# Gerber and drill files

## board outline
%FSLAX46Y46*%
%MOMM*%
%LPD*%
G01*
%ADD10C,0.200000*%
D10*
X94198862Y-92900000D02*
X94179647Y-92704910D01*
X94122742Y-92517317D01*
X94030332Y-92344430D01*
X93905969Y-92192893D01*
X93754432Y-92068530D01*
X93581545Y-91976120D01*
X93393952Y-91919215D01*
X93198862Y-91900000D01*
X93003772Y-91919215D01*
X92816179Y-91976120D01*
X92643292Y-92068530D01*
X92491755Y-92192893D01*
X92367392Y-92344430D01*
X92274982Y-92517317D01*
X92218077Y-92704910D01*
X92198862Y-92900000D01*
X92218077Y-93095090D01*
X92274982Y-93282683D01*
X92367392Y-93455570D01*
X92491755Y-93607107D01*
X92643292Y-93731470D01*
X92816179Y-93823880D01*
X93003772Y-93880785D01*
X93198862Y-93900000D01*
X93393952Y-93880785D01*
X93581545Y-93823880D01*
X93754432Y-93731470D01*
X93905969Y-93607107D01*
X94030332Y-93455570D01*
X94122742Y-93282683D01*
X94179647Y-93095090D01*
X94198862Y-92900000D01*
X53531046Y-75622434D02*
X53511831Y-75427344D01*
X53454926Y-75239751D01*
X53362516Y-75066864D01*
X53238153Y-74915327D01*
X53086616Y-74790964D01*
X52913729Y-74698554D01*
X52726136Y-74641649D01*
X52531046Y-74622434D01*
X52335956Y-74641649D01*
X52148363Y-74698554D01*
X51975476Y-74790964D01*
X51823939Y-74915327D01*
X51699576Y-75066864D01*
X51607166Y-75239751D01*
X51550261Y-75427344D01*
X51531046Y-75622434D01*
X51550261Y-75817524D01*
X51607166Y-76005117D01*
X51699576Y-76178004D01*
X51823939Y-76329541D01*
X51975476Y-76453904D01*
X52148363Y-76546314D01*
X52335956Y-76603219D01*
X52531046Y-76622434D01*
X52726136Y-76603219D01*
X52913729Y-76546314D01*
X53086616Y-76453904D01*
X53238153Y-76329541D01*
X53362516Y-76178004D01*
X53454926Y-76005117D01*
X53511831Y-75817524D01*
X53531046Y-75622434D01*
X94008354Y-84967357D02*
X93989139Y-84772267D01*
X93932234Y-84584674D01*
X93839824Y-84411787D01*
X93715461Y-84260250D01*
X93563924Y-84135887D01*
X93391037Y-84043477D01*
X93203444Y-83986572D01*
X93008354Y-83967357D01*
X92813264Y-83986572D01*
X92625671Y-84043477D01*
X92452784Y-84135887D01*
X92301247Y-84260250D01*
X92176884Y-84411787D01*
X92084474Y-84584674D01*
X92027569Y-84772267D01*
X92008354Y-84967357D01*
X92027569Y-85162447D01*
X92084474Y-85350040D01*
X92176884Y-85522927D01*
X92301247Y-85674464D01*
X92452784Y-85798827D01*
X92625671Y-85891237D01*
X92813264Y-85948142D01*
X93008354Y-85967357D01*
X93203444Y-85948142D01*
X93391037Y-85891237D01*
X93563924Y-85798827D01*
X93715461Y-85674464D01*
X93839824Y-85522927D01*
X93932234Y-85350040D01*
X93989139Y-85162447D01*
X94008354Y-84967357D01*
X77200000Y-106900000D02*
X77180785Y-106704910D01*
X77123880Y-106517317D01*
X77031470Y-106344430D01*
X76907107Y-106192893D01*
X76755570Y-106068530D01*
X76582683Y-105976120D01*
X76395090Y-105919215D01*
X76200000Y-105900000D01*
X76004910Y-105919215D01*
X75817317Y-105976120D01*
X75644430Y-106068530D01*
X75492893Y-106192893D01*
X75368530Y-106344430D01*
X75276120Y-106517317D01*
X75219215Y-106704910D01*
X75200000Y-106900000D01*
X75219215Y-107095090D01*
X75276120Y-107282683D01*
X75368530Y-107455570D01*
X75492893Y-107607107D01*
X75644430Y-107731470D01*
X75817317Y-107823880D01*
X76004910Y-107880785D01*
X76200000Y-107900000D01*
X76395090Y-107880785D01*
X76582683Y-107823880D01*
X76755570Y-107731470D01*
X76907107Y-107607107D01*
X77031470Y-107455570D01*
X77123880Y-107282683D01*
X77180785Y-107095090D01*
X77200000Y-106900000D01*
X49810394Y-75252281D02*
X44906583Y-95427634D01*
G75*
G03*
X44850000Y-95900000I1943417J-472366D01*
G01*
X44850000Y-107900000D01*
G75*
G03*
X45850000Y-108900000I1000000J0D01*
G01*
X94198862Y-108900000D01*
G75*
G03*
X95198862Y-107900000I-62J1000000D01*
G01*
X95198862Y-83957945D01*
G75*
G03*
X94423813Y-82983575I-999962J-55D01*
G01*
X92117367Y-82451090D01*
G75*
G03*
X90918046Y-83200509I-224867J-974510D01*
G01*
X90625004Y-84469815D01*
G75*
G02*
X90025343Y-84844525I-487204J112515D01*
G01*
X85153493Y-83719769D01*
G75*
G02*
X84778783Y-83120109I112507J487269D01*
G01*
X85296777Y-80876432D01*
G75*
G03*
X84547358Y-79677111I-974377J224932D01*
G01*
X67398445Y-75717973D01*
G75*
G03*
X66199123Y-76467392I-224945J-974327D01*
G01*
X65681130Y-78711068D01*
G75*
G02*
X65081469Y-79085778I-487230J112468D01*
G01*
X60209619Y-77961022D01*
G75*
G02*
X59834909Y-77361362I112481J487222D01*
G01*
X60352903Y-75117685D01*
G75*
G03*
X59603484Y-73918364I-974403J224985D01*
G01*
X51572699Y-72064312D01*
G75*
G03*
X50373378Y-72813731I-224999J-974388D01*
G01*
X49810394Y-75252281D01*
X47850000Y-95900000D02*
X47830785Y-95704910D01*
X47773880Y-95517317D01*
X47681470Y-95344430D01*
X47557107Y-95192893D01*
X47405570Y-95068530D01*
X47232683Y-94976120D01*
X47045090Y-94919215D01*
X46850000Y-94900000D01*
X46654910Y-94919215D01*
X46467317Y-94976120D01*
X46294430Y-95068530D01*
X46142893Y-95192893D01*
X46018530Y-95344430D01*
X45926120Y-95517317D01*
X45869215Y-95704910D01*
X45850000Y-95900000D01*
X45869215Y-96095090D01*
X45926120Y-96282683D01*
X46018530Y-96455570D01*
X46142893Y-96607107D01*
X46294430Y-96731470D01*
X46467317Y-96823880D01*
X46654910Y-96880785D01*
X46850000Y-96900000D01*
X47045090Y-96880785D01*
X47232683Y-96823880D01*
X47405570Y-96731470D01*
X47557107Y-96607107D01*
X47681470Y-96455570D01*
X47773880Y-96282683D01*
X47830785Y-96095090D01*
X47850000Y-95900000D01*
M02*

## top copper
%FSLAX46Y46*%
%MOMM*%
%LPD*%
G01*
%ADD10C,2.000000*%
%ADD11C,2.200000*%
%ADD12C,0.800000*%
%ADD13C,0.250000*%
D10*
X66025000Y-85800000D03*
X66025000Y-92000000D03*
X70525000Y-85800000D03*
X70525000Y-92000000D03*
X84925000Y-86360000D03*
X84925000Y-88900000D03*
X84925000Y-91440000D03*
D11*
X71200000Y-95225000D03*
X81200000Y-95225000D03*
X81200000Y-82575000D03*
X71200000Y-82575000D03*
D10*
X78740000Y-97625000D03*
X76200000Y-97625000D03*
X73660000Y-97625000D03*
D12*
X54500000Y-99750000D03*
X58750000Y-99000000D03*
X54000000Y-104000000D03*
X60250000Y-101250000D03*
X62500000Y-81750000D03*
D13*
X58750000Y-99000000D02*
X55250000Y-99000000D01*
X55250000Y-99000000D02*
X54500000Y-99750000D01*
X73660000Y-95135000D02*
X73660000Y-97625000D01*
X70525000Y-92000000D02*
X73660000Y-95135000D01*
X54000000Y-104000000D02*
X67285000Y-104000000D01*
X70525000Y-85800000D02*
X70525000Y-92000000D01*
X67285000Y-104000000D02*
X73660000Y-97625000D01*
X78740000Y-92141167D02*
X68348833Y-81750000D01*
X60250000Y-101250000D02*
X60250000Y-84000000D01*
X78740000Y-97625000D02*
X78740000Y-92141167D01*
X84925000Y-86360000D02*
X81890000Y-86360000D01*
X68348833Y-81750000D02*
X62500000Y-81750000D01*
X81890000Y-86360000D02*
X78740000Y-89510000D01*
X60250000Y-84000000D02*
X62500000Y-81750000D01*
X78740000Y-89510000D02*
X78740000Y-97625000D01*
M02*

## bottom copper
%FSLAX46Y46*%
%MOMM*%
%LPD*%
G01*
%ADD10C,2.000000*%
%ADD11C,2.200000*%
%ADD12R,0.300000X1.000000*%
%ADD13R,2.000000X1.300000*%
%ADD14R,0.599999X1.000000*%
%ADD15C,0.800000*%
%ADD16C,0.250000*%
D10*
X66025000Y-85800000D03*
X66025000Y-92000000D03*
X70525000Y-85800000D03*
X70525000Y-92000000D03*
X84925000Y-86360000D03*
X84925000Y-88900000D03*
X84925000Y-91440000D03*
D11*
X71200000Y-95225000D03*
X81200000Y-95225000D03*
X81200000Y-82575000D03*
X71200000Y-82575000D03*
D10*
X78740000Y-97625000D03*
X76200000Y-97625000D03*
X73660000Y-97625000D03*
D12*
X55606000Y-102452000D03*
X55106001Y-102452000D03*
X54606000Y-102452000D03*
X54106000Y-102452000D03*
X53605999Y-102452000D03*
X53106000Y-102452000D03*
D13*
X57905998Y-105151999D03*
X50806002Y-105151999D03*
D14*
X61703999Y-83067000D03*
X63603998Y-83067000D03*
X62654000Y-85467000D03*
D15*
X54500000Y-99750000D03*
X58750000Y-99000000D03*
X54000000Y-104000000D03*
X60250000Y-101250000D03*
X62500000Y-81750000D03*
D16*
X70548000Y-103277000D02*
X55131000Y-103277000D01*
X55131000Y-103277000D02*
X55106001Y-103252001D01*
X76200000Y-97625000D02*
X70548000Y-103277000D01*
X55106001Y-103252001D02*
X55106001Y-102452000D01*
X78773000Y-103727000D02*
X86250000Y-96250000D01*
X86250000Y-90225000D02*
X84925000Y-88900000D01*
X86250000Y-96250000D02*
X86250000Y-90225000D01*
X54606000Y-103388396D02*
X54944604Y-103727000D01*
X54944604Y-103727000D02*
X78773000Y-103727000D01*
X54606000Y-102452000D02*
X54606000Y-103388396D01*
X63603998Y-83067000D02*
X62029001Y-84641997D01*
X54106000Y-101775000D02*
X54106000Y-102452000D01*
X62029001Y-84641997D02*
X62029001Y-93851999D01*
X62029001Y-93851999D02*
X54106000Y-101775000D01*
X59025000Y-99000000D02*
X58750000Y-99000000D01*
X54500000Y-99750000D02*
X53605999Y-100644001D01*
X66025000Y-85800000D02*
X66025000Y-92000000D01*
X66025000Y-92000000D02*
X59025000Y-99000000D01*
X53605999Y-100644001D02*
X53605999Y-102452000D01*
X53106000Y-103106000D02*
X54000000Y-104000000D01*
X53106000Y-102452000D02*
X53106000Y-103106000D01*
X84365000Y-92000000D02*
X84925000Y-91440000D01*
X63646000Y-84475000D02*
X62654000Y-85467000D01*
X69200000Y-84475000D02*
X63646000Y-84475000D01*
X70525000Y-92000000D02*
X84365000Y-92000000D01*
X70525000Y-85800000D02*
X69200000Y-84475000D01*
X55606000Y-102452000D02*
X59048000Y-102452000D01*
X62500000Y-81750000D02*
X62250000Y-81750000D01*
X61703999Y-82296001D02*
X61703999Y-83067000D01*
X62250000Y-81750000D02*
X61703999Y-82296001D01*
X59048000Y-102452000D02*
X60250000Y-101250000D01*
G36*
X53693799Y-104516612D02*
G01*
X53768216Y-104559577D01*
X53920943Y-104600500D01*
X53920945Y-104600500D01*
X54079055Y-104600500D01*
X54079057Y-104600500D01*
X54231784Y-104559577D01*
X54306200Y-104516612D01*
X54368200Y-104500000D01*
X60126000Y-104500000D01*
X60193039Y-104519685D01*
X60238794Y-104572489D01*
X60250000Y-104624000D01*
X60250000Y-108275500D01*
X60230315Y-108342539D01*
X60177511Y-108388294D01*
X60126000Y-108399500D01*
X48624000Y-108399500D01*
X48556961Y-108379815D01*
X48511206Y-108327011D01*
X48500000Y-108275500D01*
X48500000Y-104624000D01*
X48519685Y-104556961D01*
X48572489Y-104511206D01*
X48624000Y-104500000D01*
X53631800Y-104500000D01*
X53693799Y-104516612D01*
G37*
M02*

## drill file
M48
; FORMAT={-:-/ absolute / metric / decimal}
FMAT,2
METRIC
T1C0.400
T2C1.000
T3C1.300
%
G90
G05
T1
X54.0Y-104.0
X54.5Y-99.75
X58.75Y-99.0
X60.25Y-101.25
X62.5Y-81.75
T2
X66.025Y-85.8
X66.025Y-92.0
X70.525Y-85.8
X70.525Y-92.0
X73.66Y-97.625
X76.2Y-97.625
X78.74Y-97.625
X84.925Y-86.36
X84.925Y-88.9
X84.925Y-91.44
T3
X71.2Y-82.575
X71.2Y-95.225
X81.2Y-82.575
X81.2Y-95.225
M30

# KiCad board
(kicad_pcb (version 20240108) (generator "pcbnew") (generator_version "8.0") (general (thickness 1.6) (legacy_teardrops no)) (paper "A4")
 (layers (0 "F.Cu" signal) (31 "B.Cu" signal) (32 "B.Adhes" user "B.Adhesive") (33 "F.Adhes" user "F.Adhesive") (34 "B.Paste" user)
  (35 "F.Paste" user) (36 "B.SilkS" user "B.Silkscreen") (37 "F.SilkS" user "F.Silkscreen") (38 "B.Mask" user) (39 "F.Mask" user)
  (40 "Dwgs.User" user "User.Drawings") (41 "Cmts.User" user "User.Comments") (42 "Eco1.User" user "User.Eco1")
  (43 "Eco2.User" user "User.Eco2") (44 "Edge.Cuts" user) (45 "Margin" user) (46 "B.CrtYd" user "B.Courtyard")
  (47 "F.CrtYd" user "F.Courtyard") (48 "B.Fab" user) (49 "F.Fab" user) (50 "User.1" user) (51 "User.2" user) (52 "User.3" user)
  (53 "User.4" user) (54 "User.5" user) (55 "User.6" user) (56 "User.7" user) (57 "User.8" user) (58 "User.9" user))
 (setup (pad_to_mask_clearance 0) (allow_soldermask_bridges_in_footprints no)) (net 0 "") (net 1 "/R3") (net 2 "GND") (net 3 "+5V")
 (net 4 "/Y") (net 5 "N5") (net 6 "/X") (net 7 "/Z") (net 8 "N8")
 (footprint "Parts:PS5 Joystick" (layer "F.Cu") (at 76.2 88.9)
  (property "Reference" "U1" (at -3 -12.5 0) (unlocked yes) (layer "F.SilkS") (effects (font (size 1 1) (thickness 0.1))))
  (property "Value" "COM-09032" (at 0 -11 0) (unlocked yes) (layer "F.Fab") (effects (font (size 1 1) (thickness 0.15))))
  (pad "B1A" thru_hole circle (at -10.175 -3.1) (size 2 2) (drill 1) (layers "*.Cu" "*.Mask") (remove_unused_layers no) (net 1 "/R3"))
  (pad "B1A" thru_hole circle (at -10.175 3.1) (size 2 2) (drill 1) (layers "*.Cu" "*.Mask") (remove_unused_layers no) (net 1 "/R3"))
  (pad "B2A" thru_hole circle (at -5.675 -3.1) (size 2 2) (drill 1) (layers "*.Cu" "*.Mask") (remove_unused_layers no) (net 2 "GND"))
  (pad "B2A" thru_hole circle (at -5.675 3.1) (size 2 2) (drill 1) (layers "*.Cu" "*.Mask") (remove_unused_layers no) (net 2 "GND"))
  (pad "H1" thru_hole circle (at 8.725 -2.54) (size 2 2) (drill 1) (layers "*.Cu" "*.Mask") (remove_unused_layers no) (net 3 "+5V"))
  (pad "H2" thru_hole circle (at 8.725 0) (size 2 2) (drill 1) (layers "*.Cu" "*.Mask") (remove_unused_layers no) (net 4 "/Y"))
  (pad "H3" thru_hole circle (at 8.725 2.54) (size 2 2) (drill 1) (layers "*.Cu" "*.Mask") (remove_unused_layers no) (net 2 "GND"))
  (pad "S1" thru_hole circle (at -5 6.325) (size 2.2 2.2) (drill 1.3) (layers "*.Cu" "*.Mask") (remove_unused_layers no) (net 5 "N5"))
  (pad "S2" thru_hole circle (at 5 6.325) (size 2.2 2.2) (drill 1.3) (layers "*.Cu" "*.Mask") (remove_unused_layers no) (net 5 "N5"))
  (pad "S3" thru_hole circle (at 5 -6.325) (size 2.2 2.2) (drill 1.3) (layers "*.Cu" "*.Mask") (remove_unused_layers no) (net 5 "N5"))
  (pad "S4" thru_hole circle (at -5 -6.325) (size 2.2 2.2) (drill 1.3) (layers "*.Cu" "*.Mask") (remove_unused_layers no) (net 5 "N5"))
  (pad "V1" thru_hole circle (at 2.54 8.725) (size 2 2) (drill 1) (layers "*.Cu" "*.Mask") (remove_unused_layers no) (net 3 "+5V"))
  (pad "V2" thru_hole circle (at 0 8.725) (size 2 2) (drill 1) (layers "*.Cu" "*.Mask") (remove_unused_layers no) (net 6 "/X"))
  (pad "V3" thru_hole circle (at -2.54 8.725) (size 2 2) (drill 1) (layers "*.Cu" "*.Mask") (remove_unused_layers no) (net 2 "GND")))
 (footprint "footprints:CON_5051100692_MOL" (layer "B.Cu") (at 54.356 104.902 180)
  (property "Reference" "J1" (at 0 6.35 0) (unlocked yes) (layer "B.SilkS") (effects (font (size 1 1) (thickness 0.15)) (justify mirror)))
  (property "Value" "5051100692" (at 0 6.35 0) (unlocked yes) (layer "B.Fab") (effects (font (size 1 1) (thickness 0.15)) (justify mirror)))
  (pad "1" smd rect (at -1.25 2.45 180) (size 0.3 1) (layers "B.Cu" "B.Paste" "B.Mask") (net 3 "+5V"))
  (pad "2" smd rect (at -0.750001 2.45 180) (size 0.3 1) (layers "B.Cu" "B.Paste" "B.Mask") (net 6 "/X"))
  (pad "3" smd rect (at -0.25 2.45 180) (size 0.3 1) (layers "B.Cu" "B.Paste" "B.Mask") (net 4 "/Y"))
  (pad "4" smd rect (at 0.25 2.45 180) (size 0.3 1) (layers "B.Cu" "B.Paste" "B.Mask") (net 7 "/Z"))
  (pad "5" smd rect (at 0.750001 2.45 180) (size 0.3 1) (layers "B.Cu" "B.Paste" "B.Mask") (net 1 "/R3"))
  (pad "6" smd rect (at 1.25 2.45 180) (size 0.3 1) (layers "B.Cu" "B.Paste" "B.Mask") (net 2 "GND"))
  (pad "P1" smd rect (at -3.549998 -0.249999 180) (size 2 1.3) (layers "B.Cu" "B.Paste" "B.Mask") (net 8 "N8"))
  (pad "P2" smd rect (at 3.549998 -0.249999 180) (size 2 1.3) (layers "B.Cu" "B.Paste" "B.Mask") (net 8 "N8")))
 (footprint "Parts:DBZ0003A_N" (layer "B.Cu") (at 62.654 84.267 -90)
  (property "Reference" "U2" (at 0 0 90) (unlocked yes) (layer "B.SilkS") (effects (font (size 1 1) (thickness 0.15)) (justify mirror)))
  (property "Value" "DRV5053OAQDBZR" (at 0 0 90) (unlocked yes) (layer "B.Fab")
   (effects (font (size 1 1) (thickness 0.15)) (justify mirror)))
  (pad "1" smd rect (at -1.2 0.950001 180) (size 0.599999 1) (layers "B.Cu" "B.Paste" "B.Mask") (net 3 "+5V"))
  (pad "2" smd rect (at -1.2 -0.949998 180) (size 0.599999 1) (layers "B.Cu" "B.Paste" "B.Mask") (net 7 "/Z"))
  (pad "3" smd rect (at 1.2 0 180) (size 0.599999 1) (layers "B.Cu" "B.Paste" "B.Mask") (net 2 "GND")))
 (gr_poly
  (pts (xy 94.198862 92.9) (xy 94.179647 92.70491) (xy 94.122742 92.517317) (xy 94.030332 92.34443) (xy 93.905969 92.192893)
   (xy 93.754432 92.06853) (xy 93.581545 91.97612) (xy 93.393952 91.919215) (xy 93.198862 91.9) (xy 93.003772 91.919215)
   (xy 92.816179 91.97612) (xy 92.643292 92.06853) (xy 92.491755 92.192893) (xy 92.367392 92.34443) (xy 92.274982 92.517317)
   (xy 92.218077 92.70491) (xy 92.198862 92.9) (xy 92.218077 93.09509) (xy 92.274982 93.282683) (xy 92.367392 93.45557)
   (xy 92.491755 93.607107) (xy 92.643292 93.73147) (xy 92.816179 93.82388) (xy 93.003772 93.880785) (xy 93.198862 93.9)
   (xy 93.393952 93.880785) (xy 93.581545 93.82388) (xy 93.754432 93.73147) (xy 93.905969 93.607107) (xy 94.030332 93.45557)
   (xy 94.122742 93.282683) (xy 94.179647 93.09509) (xy 94.198862 92.9))
  (stroke (width 0.2) (type solid)) (fill none) (layer "Edge.Cuts"))
 (gr_poly
  (pts (xy 53.531046 75.622434) (xy 53.511831 75.427344) (xy 53.454926 75.239751) (xy 53.362516 75.066864) (xy 53.238153 74.915327)
   (xy 53.086616 74.790964) (xy 52.913729 74.698554) (xy 52.726136 74.641649) (xy 52.531046 74.622434) (xy 52.335956 74.641649)
   (xy 52.148363 74.698554) (xy 51.975476 74.790964) (xy 51.823939 74.915327) (xy 51.699576 75.066864) (xy 51.607166 75.239751)
   (xy 51.550261 75.427344) (xy 51.531046 75.622434) (xy 51.550261 75.817524) (xy 51.607166 76.005117) (xy 51.699576 76.178004)
   (xy 51.823939 76.329541) (xy 51.975476 76.453904) (xy 52.148363 76.546314) (xy 52.335956 76.603219) (xy 52.531046 76.622434)
   (xy 52.726136 76.603219) (xy 52.913729 76.546314) (xy 53.086616 76.453904) (xy 53.238153 76.329541) (xy 53.362516 76.178004)
   (xy 53.454926 76.005117) (xy 53.511831 75.817524) (xy 53.531046 75.622434))
  (stroke (width 0.2) (type solid)) (fill none) (layer "Edge.Cuts"))
 (gr_poly
  (pts (xy 94.008354 84.967357) (xy 93.989139 84.772267) (xy 93.932234 84.584674) (xy 93.839824 84.411787) (xy 93.715461 84.26025)
   (xy 93.563924 84.135887) (xy 93.391037 84.043477) (xy 93.203444 83.986572) (xy 93.008354 83.967357) (xy 92.813264 83.986572)
   (xy 92.625671 84.043477) (xy 92.452784 84.135887) (xy 92.301247 84.26025) (xy 92.176884 84.411787) (xy 92.084474 84.584674)
   (xy 92.027569 84.772267) (xy 92.008354 84.967357) (xy 92.027569 85.162447) (xy 92.084474 85.35004) (xy 92.176884 85.522927)
   (xy 92.301247 85.674464) (xy 92.452784 85.798827) (xy 92.625671 85.891237) (xy 92.813264 85.948142) (xy 93.008354 85.967357)
   (xy 93.203444 85.948142) (xy 93.391037 85.891237) (xy 93.563924 85.798827) (xy 93.715461 85.674464) (xy 93.839824 85.522927)
   (xy 93.932234 85.35004) (xy 93.989139 85.162447) (xy 94.008354 84.967357))
  (stroke (width 0.2) (type solid)) (fill none) (layer "Edge.Cuts"))
 (gr_poly
  (pts (xy 77.2 106.9) (xy 77.180785 106.70491) (xy 77.12388 106.517317) (xy 77.03147 106.34443) (xy 76.907107 106.192893)
   (xy 76.75557 106.06853) (xy 76.582683 105.97612) (xy 76.39509 105.919215) (xy 76.2 105.9) (xy 76.00491 105.919215)
   (xy 75.817317 105.97612) (xy 75.64443 106.06853) (xy 75.492893 106.192893) (xy 75.36853 106.34443) (xy 75.27612 106.517317)
   (xy 75.219215 106.70491) (xy 75.2 106.9) (xy 75.219215 107.09509) (xy 75.27612 107.282683) (xy 75.36853 107.45557)
   (xy 75.492893 107.607107) (xy 75.64443 107.73147) (xy 75.817317 107.82388) (xy 76.00491 107.880785) (xy 76.2 107.9)
   (xy 76.39509 107.880785) (xy 76.582683 107.82388) (xy 76.75557 107.73147) (xy 76.907107 107.607107) (xy 77.03147 107.45557)
   (xy 77.12388 107.282683) (xy 77.180785 107.09509) (xy 77.2 106.9))
  (stroke (width 0.2) (type solid)) (fill none) (layer "Edge.Cuts"))
 (gr_poly
  (pts (xy 49.810394 75.252281)
   (arc (start 44.906583 95.427634) (mid 44.864196 95.662129) (end 44.85 95.9))
   (arc (start 44.85 107.9) (mid 45.142893 108.607107) (end 45.85 108.9))
   (arc (start 94.198862 108.9) (mid 94.905966 108.607093) (end 95.198862 107.9))
   (arc (start 95.198862 83.957945) (mid 94.981467 83.335431) (end 94.423813 82.983575))
   (arc (start 92.117367 82.45109) (mid 91.362505 82.577445) (end 90.918046 83.200509))
   (arc (start 90.625004 84.469815) (mid 90.402771 84.781349) (end 90.025343 84.844525))
   (arc (start 85.153493 83.719769) (mid 84.841972 83.497537) (end 84.778783 83.120109))
   (arc (start 85.296777 80.876432) (mid 85.170456 80.121561) (end 84.547358 79.677111))
   (arc (start 67.398445 75.717973) (mid 66.643574 75.844295) (end 66.199123 76.467392))
   (arc (start 65.68113 78.711068) (mid 65.458904 79.022617) (end 65.081469 79.085778))
   (arc (start 60.209619 77.961022) (mid 59.89807 77.738797) (end 59.834909 77.361362))
   (arc (start 60.352903 75.117685) (mid 60.226581 74.362815) (end 59.603484 73.918364))
   (arc (start 51.572699 72.064312) (mid 50.817829 72.190634) (end 50.373378 72.813731)))
  (stroke (width 0.2) (type solid)) (fill none) (layer "Edge.Cuts"))
 (gr_poly
  (pts (xy 47.85 95.9) (xy 47.830785 95.70491) (xy 47.77388 95.517317) (xy 47.68147 95.34443) (xy 47.557107 95.192893)
   (xy 47.40557 95.06853) (xy 47.232683 94.97612) (xy 47.04509 94.919215) (xy 46.85 94.9) (xy 46.65491 94.919215) (xy 46.467317 94.97612)
   (xy 46.29443 95.06853) (xy 46.142893 95.192893) (xy 46.01853 95.34443) (xy 45.92612 95.517317) (xy 45.869215 95.70491) (xy 45.85 95.9)
   (xy 45.869215 96.09509) (xy 45.92612 96.282683) (xy 46.01853 96.45557) (xy 46.142893 96.607107) (xy 46.29443 96.73147)
   (xy 46.467317 96.82388) (xy 46.65491 96.880785) (xy 46.85 96.9) (xy 47.04509 96.880785) (xy 47.232683 96.82388) (xy 47.40557 96.73147)
   (xy 47.557107 96.607107) (xy 47.68147 96.45557) (xy 47.77388 96.282683) (xy 47.830785 96.09509) (xy 47.85 95.9))
  (stroke (width 0.2) (type solid)) (fill none) (layer "Edge.Cuts"))
 (segment (start 70.548 103.277) (end 55.131 103.277) (width 0.25) (layer "B.Cu") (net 6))
 (segment (start 55.131 103.277) (end 55.106001 103.252001) (width 0.25) (layer "B.Cu") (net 6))
 (segment (start 76.2 97.625) (end 70.548 103.277) (width 0.25) (layer "B.Cu") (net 6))
 (segment (start 55.106001 103.252001) (end 55.106001 102.452) (width 0.25) (layer "B.Cu") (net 6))
 (segment (start 78.773 103.727) (end 86.25 96.25) (width 0.25) (layer "B.Cu") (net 4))
 (segment (start 86.25 90.225) (end 84.925 88.9) (width 0.25) (layer "B.Cu") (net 4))
 (segment (start 86.25 96.25) (end 86.25 90.225) (width 0.25) (layer "B.Cu") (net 4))
 (segment (start 54.606 103.388396) (end 54.944604 103.727) (width 0.25) (layer "B.Cu") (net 4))
 (segment (start 54.944604 103.727) (end 78.773 103.727) (width 0.25) (layer "B.Cu") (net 4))
 (segment (start 54.606 102.452) (end 54.606 103.388396) (width 0.25) (layer "B.Cu") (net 4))
 (segment (start 63.603998 83.067) (end 62.029001 84.641997) (width 0.25) (layer "B.Cu") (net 7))
 (segment (start 54.106 101.775) (end 54.106 102.452) (width 0.25) (layer "B.Cu") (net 7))
 (segment (start 62.029001 84.641997) (end 62.029001 93.851999) (width 0.25) (layer "B.Cu") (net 7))
 (segment (start 62.029001 93.851999) (end 54.106 101.775) (width 0.25) (layer "B.Cu") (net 7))
 (segment (start 58.75 99) (end 55.25 99) (width 0.25) (layer "F.Cu") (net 1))
 (segment (start 55.25 99) (end 54.5 99.75) (width 0.25) (layer "F.Cu") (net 1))
 (via (at 54.5 99.75) (size 0.8) (drill 0.4) (layers "F.Cu" "B.Cu") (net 1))
 (via (at 58.75 99) (size 0.8) (drill 0.4) (layers "F.Cu" "B.Cu") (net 1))
 (segment (start 59.025 99) (end 58.75 99) (width 0.25) (layer "B.Cu") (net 1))
 (segment (start 54.5 99.75) (end 53.605999 100.644001) (width 0.25) (layer "B.Cu") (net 1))
 (segment (start 66.025 85.8) (end 66.025 92) (width 0.25) (layer "B.Cu") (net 1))
 (segment (start 66.025 92) (end 59.025 99) (width 0.25) (layer "B.Cu") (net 1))
 (segment (start 53.605999 100.644001) (end 53.605999 102.452) (width 0.25) (layer "B.Cu") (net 1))
 (segment (start 73.66 95.135) (end 73.66 97.625) (width 0.25) (layer "F.Cu") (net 2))
 (segment (start 70.525 92) (end 73.66 95.135) (width 0.25) (layer "F.Cu") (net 2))
 (segment (start 54 104) (end 67.285 104) (width 0.25) (layer "F.Cu") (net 2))
 (segment (start 70.525 85.8) (end 70.525 92) (width 0.25) (layer "F.Cu") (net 2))
 (segment (start 67.285 104) (end 73.66 97.625) (width 0.25) (layer "F.Cu") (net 2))
 (via (at 54 104) (size 0.8) (drill 0.4) (layers "F.Cu" "B.Cu") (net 2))
 (segment (start 53.106 103.106) (end 54 104) (width 0.25) (layer "B.Cu") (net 2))
 (segment (start 53.106 102.452) (end 53.106 103.106) (width 0.25) (layer "B.Cu") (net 2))
 (segment (start 84.365 92) (end 84.925 91.44) (width 0.25) (layer "B.Cu") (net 2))
 (segment (start 63.646 84.475) (end 62.654 85.467) (width 0.25) (layer "B.Cu") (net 2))
 (segment (start 69.2 84.475) (end 63.646 84.475) (width 0.25) (layer "B.Cu") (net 2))
 (segment (start 70.525 92) (end 84.365 92) (width 0.25) (layer "B.Cu") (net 2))
 (segment (start 70.525 85.8) (end 69.2 84.475) (width 0.25) (layer "B.Cu") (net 2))
 (segment (start 78.74 92.141167) (end 68.348833 81.75) (width 0.25) (layer "F.Cu") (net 3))
 (segment (start 60.25 101.25) (end 60.25 84) (width 0.25) (layer "F.Cu") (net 3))
 (segment (start 78.74 97.625) (end 78.74 92.141167) (width 0.25) (layer "F.Cu") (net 3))
 (segment (start 84.925 86.36) (end 81.89 86.36) (width 0.25) (layer "F.Cu") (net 3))
 (segment (start 68.348833 81.75) (end 62.5 81.75) (width 0.25) (layer "F.Cu") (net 3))
 (segment (start 81.89 86.36) (end 78.74 89.51) (width 0.25) (layer "F.Cu") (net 3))
 (segment (start 60.25 84) (end 62.5 81.75) (width 0.25) (layer "F.Cu") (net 3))
 (segment (start 78.74 89.51) (end 78.74 97.625) (width 0.25) (layer "F.Cu") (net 3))
 (via (at 60.25 101.25) (size 0.8) (drill 0.4) (layers "F.Cu" "B.Cu") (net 3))
 (via (at 62.5 81.75) (size 0.8) (drill 0.4) (layers "F.Cu" "B.Cu") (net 3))
 (segment (start 55.606 102.452) (end 59.048 102.452) (width 0.25) (layer "B.Cu") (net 3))
 (segment (start 62.5 81.75) (end 62.25 81.75) (width 0.25) (layer "B.Cu") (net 3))
 (segment (start 61.703999 82.296001) (end 61.703999 83.067) (width 0.25) (layer "B.Cu") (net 3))
 (segment (start 62.25 81.75) (end 61.703999 82.296001) (width 0.25) (layer "B.Cu") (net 3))
 (segment (start 59.048 102.452) (end 60.25 101.25) (width 0.25) (layer "B.Cu") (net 3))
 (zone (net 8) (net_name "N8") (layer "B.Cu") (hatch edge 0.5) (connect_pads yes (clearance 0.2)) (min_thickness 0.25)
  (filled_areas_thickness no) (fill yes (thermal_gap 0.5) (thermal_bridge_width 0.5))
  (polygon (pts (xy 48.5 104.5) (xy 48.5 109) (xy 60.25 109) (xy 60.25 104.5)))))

